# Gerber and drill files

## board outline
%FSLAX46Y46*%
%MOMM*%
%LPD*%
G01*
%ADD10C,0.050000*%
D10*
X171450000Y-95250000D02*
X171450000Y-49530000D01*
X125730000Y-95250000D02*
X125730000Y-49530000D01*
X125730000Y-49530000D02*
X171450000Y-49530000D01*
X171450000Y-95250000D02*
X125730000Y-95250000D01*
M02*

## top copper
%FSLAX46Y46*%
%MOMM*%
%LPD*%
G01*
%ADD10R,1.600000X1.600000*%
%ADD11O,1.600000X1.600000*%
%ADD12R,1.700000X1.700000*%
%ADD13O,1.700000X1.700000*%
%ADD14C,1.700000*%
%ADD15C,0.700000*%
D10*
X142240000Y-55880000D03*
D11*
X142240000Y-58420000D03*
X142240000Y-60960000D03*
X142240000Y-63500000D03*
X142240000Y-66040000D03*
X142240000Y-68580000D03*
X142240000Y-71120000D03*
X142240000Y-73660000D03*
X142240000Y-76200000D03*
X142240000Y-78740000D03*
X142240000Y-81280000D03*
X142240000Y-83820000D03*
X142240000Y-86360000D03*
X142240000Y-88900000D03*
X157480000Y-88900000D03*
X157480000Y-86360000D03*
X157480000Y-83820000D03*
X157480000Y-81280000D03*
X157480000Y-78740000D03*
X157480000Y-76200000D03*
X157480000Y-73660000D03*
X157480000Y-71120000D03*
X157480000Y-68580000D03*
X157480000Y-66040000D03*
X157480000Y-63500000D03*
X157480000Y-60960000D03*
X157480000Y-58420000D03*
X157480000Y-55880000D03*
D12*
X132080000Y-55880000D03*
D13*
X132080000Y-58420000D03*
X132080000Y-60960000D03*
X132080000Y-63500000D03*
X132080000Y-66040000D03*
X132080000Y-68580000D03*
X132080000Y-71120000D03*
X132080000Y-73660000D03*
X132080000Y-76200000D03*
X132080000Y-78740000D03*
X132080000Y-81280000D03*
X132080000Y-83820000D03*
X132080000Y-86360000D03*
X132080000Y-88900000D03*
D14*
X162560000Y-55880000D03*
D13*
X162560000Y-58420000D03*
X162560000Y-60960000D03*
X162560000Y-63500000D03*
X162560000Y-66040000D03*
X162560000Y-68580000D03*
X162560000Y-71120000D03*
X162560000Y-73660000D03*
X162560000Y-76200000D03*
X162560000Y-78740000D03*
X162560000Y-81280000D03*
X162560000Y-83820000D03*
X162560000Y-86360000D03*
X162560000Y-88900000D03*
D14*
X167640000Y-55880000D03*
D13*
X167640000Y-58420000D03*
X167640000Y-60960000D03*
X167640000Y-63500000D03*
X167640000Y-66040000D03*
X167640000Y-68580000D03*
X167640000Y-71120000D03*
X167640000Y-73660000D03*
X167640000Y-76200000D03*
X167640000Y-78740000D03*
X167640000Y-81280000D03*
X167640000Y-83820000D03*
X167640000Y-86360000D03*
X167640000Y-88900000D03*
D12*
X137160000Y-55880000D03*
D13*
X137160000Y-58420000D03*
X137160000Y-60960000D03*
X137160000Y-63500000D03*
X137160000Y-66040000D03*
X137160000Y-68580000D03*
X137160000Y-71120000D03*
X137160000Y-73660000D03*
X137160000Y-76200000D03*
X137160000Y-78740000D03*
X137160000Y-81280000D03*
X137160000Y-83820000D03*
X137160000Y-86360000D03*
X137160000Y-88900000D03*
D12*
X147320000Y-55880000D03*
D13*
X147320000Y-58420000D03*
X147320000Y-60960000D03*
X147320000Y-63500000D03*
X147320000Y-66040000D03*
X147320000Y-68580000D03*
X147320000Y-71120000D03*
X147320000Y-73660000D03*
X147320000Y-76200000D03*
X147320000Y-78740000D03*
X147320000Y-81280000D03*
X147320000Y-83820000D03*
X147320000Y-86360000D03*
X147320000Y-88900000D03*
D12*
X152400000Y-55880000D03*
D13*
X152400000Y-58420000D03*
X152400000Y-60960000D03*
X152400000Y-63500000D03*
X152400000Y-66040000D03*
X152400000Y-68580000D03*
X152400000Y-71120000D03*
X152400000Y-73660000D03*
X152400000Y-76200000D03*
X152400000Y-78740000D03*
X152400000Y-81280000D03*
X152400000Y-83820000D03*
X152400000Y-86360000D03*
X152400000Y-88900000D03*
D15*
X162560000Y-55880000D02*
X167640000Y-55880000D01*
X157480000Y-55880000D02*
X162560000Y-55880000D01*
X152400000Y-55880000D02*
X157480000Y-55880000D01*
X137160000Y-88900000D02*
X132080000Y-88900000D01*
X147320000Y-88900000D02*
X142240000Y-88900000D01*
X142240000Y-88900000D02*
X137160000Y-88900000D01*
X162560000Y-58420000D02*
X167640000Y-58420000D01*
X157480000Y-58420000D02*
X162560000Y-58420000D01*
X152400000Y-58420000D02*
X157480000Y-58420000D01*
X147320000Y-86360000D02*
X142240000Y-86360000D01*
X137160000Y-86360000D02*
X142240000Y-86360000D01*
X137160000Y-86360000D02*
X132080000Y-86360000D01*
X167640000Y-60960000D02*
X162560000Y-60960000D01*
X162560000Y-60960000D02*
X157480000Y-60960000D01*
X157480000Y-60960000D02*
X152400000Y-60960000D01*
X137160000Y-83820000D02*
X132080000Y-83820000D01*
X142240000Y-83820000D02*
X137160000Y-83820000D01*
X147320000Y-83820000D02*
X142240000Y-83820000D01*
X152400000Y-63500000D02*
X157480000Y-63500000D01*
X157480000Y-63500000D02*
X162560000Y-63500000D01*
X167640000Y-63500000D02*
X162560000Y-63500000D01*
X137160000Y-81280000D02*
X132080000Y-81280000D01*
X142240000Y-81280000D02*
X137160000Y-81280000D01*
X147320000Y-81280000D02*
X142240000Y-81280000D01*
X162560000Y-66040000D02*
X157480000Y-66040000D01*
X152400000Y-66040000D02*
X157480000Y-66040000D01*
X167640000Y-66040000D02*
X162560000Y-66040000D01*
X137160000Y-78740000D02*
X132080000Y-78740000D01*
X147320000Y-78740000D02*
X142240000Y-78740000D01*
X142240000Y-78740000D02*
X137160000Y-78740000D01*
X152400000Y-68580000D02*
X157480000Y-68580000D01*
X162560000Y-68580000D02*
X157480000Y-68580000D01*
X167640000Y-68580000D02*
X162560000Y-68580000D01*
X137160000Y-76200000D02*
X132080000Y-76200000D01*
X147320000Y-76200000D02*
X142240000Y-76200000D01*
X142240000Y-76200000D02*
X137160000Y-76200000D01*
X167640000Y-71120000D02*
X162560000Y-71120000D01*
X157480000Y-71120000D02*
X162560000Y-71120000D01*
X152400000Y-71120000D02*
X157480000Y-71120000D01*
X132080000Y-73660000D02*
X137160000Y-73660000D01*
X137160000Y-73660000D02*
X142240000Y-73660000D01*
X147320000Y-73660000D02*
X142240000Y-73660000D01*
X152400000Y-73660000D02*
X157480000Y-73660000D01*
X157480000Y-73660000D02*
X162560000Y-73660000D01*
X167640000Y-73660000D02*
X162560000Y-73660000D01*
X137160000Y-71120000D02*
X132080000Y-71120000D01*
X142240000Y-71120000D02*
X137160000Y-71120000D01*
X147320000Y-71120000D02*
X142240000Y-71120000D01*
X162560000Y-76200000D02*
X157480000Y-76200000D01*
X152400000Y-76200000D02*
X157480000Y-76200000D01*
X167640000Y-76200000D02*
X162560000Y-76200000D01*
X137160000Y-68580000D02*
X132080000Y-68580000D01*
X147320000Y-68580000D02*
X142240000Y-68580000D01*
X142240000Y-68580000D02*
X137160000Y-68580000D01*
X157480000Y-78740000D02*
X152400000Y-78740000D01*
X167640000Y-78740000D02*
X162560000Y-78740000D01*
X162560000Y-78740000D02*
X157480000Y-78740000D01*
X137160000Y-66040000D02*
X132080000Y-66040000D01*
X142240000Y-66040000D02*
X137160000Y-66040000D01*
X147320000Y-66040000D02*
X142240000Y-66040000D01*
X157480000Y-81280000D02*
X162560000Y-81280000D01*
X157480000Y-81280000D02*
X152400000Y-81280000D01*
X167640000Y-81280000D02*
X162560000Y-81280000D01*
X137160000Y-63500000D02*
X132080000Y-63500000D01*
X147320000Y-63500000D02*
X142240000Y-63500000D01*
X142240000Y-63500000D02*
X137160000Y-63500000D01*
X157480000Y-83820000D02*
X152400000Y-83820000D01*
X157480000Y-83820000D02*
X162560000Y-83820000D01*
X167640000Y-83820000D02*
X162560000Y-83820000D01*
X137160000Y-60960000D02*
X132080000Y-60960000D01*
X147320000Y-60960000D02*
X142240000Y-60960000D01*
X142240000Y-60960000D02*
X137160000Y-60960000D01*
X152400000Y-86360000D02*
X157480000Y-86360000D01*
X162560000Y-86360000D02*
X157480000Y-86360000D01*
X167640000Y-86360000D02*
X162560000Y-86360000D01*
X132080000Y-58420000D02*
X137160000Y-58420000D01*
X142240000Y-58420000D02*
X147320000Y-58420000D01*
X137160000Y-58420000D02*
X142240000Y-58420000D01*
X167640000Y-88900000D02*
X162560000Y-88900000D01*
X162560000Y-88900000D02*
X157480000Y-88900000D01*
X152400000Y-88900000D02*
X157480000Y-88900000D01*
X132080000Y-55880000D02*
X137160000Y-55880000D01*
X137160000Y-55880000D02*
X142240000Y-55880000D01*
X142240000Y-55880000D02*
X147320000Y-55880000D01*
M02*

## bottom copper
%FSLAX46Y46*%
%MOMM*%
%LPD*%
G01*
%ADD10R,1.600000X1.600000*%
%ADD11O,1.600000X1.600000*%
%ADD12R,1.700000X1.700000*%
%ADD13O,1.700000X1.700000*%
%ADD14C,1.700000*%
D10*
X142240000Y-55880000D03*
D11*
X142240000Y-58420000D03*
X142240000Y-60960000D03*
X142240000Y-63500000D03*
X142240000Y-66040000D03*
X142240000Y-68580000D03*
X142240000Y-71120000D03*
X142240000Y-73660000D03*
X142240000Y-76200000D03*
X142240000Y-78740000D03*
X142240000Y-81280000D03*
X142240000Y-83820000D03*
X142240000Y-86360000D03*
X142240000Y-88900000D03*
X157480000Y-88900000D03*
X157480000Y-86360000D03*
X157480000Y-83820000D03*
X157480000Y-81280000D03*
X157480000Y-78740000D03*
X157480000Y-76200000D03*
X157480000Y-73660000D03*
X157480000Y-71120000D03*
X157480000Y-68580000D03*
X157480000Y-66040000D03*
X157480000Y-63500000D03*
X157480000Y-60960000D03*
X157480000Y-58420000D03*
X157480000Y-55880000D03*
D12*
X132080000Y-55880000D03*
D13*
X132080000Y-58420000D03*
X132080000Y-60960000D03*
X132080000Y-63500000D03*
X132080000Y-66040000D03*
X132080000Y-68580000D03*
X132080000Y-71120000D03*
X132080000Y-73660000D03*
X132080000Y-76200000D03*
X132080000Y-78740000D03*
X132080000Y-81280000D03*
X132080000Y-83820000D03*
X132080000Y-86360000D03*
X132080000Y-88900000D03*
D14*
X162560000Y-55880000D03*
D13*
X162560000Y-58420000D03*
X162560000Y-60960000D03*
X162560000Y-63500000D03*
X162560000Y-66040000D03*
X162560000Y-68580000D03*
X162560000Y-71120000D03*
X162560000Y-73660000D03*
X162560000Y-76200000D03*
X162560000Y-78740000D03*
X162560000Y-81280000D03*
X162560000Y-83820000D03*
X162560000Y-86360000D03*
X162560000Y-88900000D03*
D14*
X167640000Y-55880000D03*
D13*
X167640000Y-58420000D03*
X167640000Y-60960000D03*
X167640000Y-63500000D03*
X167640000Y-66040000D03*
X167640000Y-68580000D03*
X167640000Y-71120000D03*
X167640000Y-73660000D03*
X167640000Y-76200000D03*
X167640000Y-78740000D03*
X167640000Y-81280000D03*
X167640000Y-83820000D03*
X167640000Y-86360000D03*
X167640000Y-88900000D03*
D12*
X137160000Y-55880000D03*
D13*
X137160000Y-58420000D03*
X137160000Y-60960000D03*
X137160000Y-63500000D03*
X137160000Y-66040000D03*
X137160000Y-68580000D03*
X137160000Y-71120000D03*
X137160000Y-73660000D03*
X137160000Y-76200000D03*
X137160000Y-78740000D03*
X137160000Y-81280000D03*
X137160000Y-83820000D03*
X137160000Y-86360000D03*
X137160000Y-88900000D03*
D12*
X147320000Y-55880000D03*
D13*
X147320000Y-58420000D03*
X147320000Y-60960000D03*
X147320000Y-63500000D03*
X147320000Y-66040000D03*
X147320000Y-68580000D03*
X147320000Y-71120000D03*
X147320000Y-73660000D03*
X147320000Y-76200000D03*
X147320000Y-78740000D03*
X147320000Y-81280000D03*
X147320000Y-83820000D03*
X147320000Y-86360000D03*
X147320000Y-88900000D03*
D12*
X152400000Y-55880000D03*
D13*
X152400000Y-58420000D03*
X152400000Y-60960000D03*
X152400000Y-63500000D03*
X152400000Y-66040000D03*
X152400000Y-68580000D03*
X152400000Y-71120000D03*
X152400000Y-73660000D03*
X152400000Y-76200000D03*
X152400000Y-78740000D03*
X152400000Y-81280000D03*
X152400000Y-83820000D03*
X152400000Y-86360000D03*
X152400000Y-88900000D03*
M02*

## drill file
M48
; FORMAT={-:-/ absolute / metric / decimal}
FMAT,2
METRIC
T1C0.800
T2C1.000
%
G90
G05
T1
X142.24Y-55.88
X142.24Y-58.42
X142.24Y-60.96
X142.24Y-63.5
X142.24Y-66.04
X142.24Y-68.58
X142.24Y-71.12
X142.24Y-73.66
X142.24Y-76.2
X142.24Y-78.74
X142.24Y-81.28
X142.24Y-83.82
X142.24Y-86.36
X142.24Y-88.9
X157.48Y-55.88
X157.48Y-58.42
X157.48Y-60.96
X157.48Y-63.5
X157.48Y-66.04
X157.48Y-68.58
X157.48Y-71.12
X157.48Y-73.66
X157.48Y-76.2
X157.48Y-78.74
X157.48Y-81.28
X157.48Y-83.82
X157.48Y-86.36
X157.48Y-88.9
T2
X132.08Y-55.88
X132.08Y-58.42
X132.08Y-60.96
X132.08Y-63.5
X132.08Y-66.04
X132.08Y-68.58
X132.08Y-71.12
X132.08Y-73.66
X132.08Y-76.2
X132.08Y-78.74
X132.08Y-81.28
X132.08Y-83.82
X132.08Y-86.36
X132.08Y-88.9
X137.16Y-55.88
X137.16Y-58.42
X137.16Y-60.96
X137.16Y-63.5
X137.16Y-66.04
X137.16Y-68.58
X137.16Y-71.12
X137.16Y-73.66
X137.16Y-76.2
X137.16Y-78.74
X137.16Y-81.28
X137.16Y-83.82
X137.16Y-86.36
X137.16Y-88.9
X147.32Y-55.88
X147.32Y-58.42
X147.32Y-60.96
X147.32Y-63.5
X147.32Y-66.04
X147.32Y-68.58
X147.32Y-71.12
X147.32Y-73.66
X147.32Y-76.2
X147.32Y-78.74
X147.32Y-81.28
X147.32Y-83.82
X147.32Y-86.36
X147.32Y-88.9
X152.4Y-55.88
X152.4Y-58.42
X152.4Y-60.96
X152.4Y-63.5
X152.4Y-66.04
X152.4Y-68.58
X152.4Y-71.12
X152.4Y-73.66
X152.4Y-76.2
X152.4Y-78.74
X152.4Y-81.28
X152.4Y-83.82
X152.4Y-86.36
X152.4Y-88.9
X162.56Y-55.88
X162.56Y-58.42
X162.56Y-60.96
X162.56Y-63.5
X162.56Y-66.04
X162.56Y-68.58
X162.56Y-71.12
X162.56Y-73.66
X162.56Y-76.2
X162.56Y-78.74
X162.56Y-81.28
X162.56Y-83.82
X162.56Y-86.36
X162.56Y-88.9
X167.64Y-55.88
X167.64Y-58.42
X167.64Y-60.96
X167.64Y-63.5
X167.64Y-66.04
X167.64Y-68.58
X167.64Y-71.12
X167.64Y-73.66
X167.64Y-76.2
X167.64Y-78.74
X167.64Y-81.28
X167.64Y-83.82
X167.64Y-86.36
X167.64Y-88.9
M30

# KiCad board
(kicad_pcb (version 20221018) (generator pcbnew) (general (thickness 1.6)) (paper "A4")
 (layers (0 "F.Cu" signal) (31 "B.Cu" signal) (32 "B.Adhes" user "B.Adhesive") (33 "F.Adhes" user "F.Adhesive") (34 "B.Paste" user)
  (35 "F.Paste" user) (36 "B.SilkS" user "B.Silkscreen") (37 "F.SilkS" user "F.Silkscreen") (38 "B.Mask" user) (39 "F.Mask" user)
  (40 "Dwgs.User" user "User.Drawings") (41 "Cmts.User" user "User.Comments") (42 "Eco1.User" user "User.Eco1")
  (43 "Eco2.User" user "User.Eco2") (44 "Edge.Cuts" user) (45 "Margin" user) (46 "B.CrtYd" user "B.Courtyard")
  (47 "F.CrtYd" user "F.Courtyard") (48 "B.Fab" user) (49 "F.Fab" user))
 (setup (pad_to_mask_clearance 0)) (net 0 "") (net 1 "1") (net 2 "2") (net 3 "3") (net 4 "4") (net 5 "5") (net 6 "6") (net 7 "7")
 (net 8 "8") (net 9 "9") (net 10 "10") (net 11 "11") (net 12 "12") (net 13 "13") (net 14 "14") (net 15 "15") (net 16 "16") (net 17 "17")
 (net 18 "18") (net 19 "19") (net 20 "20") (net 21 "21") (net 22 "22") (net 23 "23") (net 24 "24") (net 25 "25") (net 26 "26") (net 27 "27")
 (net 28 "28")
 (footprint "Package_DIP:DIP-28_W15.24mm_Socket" (layer "F.Cu") (at 142.24 55.88)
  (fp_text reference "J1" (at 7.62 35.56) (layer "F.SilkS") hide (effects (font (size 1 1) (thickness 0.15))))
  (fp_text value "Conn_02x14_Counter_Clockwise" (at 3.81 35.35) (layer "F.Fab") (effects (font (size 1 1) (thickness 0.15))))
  (pad "1" thru_hole rect (at 0 0) (size 1.6 1.6) (drill 0.8) (layers "*.Cu" "*.Mask") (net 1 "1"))
  (pad "2" thru_hole oval (at 0 2.54) (size 1.6 1.6) (drill 0.8) (layers "*.Cu" "*.Mask") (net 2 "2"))
  (pad "3" thru_hole oval (at 0 5.08) (size 1.6 1.6) (drill 0.8) (layers "*.Cu" "*.Mask") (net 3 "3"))
  (pad "4" thru_hole oval (at 0 7.62) (size 1.6 1.6) (drill 0.8) (layers "*.Cu" "*.Mask") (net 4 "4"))
  (pad "5" thru_hole oval (at 0 10.16) (size 1.6 1.6) (drill 0.8) (layers "*.Cu" "*.Mask") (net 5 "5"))
  (pad "6" thru_hole oval (at 0 12.7) (size 1.6 1.6) (drill 0.8) (layers "*.Cu" "*.Mask") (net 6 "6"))
  (pad "7" thru_hole oval (at 0 15.24) (size 1.6 1.6) (drill 0.8) (layers "*.Cu" "*.Mask") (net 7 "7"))
  (pad "8" thru_hole oval (at 0 17.78) (size 1.6 1.6) (drill 0.8) (layers "*.Cu" "*.Mask") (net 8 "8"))
  (pad "9" thru_hole oval (at 0 20.32) (size 1.6 1.6) (drill 0.8) (layers "*.Cu" "*.Mask") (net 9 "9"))
  (pad "10" thru_hole oval (at 0 22.86) (size 1.6 1.6) (drill 0.8) (layers "*.Cu" "*.Mask") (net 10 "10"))
  (pad "11" thru_hole oval (at 0 25.4) (size 1.6 1.6) (drill 0.8) (layers "*.Cu" "*.Mask") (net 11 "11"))
  (pad "12" thru_hole oval (at 0 27.94) (size 1.6 1.6) (drill 0.8) (layers "*.Cu" "*.Mask") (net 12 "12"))
  (pad "13" thru_hole oval (at 0 30.48) (size 1.6 1.6) (drill 0.8) (layers "*.Cu" "*.Mask") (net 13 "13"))
  (pad "14" thru_hole oval (at 0 33.02) (size 1.6 1.6) (drill 0.8) (layers "*.Cu" "*.Mask") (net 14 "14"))
  (pad "15" thru_hole oval (at 15.24 33.02) (size 1.6 1.6) (drill 0.8) (layers "*.Cu" "*.Mask") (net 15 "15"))
  (pad "16" thru_hole oval (at 15.24 30.48) (size 1.6 1.6) (drill 0.8) (layers "*.Cu" "*.Mask") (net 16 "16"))
  (pad "17" thru_hole oval (at 15.24 27.94) (size 1.6 1.6) (drill 0.8) (layers "*.Cu" "*.Mask") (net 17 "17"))
  (pad "18" thru_hole oval (at 15.24 25.4) (size 1.6 1.6) (drill 0.8) (layers "*.Cu" "*.Mask") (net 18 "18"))
  (pad "19" thru_hole oval (at 15.24 22.86) (size 1.6 1.6) (drill 0.8) (layers "*.Cu" "*.Mask") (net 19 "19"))
  (pad "20" thru_hole oval (at 15.24 20.32) (size 1.6 1.6) (drill 0.8) (layers "*.Cu" "*.Mask") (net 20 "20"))
  (pad "21" thru_hole oval (at 15.24 17.78) (size 1.6 1.6) (drill 0.8) (layers "*.Cu" "*.Mask") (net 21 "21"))
  (pad "22" thru_hole oval (at 15.24 15.24) (size 1.6 1.6) (drill 0.8) (layers "*.Cu" "*.Mask") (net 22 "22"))
  (pad "23" thru_hole oval (at 15.24 12.7) (size 1.6 1.6) (drill 0.8) (layers "*.Cu" "*.Mask") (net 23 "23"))
  (pad "24" thru_hole oval (at 15.24 10.16) (size 1.6 1.6) (drill 0.8) (layers "*.Cu" "*.Mask") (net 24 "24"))
  (pad "25" thru_hole oval (at 15.24 7.62) (size 1.6 1.6) (drill 0.8) (layers "*.Cu" "*.Mask") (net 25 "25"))
  (pad "26" thru_hole oval (at 15.24 5.08) (size 1.6 1.6) (drill 0.8) (layers "*.Cu" "*.Mask") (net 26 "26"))
  (pad "27" thru_hole oval (at 15.24 2.54) (size 1.6 1.6) (drill 0.8) (layers "*.Cu" "*.Mask") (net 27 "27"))
  (pad "28" thru_hole oval (at 15.24 0) (size 1.6 1.6) (drill 0.8) (layers "*.Cu" "*.Mask") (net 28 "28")))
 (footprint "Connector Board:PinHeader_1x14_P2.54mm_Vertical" (layer "F.Cu") (at 132.08 55.88)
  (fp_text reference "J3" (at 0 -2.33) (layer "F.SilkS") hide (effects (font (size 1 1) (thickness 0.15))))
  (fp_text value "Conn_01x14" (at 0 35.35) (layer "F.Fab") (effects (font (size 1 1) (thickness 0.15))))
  (pad "1" thru_hole rect (at 0 0) (size 1.7 1.7) (drill 1) (layers "*.Cu" "*.Mask") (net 1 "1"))
  (pad "2" thru_hole oval (at 0 2.54) (size 1.7 1.7) (drill 1) (layers "*.Cu" "*.Mask") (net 2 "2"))
  (pad "3" thru_hole oval (at 0 5.08) (size 1.7 1.7) (drill 1) (layers "*.Cu" "*.Mask") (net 3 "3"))
  (pad "4" thru_hole oval (at 0 7.62) (size 1.7 1.7) (drill 1) (layers "*.Cu" "*.Mask") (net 4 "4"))
  (pad "5" thru_hole oval (at 0 10.16) (size 1.7 1.7) (drill 1) (layers "*.Cu" "*.Mask") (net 5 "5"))
  (pad "6" thru_hole oval (at 0 12.7) (size 1.7 1.7) (drill 1) (layers "*.Cu" "*.Mask") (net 6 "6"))
  (pad "7" thru_hole oval (at 0 15.24) (size 1.7 1.7) (drill 1) (layers "*.Cu" "*.Mask") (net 7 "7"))
  (pad "8" thru_hole oval (at 0 17.78) (size 1.7 1.7) (drill 1) (layers "*.Cu" "*.Mask") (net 8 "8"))
  (pad "9" thru_hole oval (at 0 20.32) (size 1.7 1.7) (drill 1) (layers "*.Cu" "*.Mask") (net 9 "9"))
  (pad "10" thru_hole oval (at 0 22.86) (size 1.7 1.7) (drill 1) (layers "*.Cu" "*.Mask") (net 10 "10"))
  (pad "11" thru_hole oval (at 0 25.4) (size 1.7 1.7) (drill 1) (layers "*.Cu" "*.Mask") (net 11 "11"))
  (pad "12" thru_hole oval (at 0 27.94) (size 1.7 1.7) (drill 1) (layers "*.Cu" "*.Mask") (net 12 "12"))
  (pad "13" thru_hole oval (at 0 30.48) (size 1.7 1.7) (drill 1) (layers "*.Cu" "*.Mask") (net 13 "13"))
  (pad "14" thru_hole oval (at 0 33.02) (size 1.7 1.7) (drill 1) (layers "*.Cu" "*.Mask") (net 14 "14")))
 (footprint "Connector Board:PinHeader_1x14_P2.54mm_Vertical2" (layer "F.Cu") (at 162.56 55.88)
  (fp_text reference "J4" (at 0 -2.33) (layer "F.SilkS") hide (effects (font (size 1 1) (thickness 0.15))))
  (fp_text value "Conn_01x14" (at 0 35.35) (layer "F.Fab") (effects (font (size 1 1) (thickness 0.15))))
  (pad "1" thru_hole circle (at 0 0) (size 1.7 1.7) (drill 1) (layers "*.Cu" "*.Mask") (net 28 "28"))
  (pad "2" thru_hole oval (at 0 2.54) (size 1.7 1.7) (drill 1) (layers "*.Cu" "*.Mask") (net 27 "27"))
  (pad "3" thru_hole oval (at 0 5.08) (size 1.7 1.7) (drill 1) (layers "*.Cu" "*.Mask") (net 26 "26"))
  (pad "4" thru_hole oval (at 0 7.62) (size 1.7 1.7) (drill 1) (layers "*.Cu" "*.Mask") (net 25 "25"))
  (pad "5" thru_hole oval (at 0 10.16) (size 1.7 1.7) (drill 1) (layers "*.Cu" "*.Mask") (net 24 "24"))
  (pad "6" thru_hole oval (at 0 12.7) (size 1.7 1.7) (drill 1) (layers "*.Cu" "*.Mask") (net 23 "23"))
  (pad "7" thru_hole oval (at 0 15.24) (size 1.7 1.7) (drill 1) (layers "*.Cu" "*.Mask") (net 22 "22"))
  (pad "8" thru_hole oval (at 0 17.78) (size 1.7 1.7) (drill 1) (layers "*.Cu" "*.Mask") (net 21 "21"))
  (pad "9" thru_hole oval (at 0 20.32) (size 1.7 1.7) (drill 1) (layers "*.Cu" "*.Mask") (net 20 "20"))
  (pad "10" thru_hole oval (at 0 22.86) (size 1.7 1.7) (drill 1) (layers "*.Cu" "*.Mask") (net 19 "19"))
  (pad "11" thru_hole oval (at 0 25.4) (size 1.7 1.7) (drill 1) (layers "*.Cu" "*.Mask") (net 18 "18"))
  (pad "12" thru_hole oval (at 0 27.94) (size 1.7 1.7) (drill 1) (layers "*.Cu" "*.Mask") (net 17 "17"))
  (pad "13" thru_hole oval (at 0 30.48) (size 1.7 1.7) (drill 1) (layers "*.Cu" "*.Mask") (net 16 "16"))
  (pad "14" thru_hole oval (at 0 33.02) (size 1.7 1.7) (drill 1) (layers "*.Cu" "*.Mask") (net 15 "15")))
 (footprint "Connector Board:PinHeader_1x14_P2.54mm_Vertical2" (layer "F.Cu") (at 167.64 55.88)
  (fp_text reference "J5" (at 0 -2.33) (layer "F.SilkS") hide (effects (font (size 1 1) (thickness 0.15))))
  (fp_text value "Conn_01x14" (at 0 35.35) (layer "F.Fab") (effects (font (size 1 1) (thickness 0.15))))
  (pad "1" thru_hole circle (at 0 0) (size 1.7 1.7) (drill 1) (layers "*.Cu" "*.Mask") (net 28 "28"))
  (pad "2" thru_hole oval (at 0 2.54) (size 1.7 1.7) (drill 1) (layers "*.Cu" "*.Mask") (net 27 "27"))
  (pad "3" thru_hole oval (at 0 5.08) (size 1.7 1.7) (drill 1) (layers "*.Cu" "*.Mask") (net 26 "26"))
  (pad "4" thru_hole oval (at 0 7.62) (size 1.7 1.7) (drill 1) (layers "*.Cu" "*.Mask") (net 25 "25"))
  (pad "5" thru_hole oval (at 0 10.16) (size 1.7 1.7) (drill 1) (layers "*.Cu" "*.Mask") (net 24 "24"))
  (pad "6" thru_hole oval (at 0 12.7) (size 1.7 1.7) (drill 1) (layers "*.Cu" "*.Mask") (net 23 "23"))
  (pad "7" thru_hole oval (at 0 15.24) (size 1.7 1.7) (drill 1) (layers "*.Cu" "*.Mask") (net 22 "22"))
  (pad "8" thru_hole oval (at 0 17.78) (size 1.7 1.7) (drill 1) (layers "*.Cu" "*.Mask") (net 21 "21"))
  (pad "9" thru_hole oval (at 0 20.32) (size 1.7 1.7) (drill 1) (layers "*.Cu" "*.Mask") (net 20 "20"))
  (pad "10" thru_hole oval (at 0 22.86) (size 1.7 1.7) (drill 1) (layers "*.Cu" "*.Mask") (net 19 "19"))
  (pad "11" thru_hole oval (at 0 25.4) (size 1.7 1.7) (drill 1) (layers "*.Cu" "*.Mask") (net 18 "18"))
  (pad "12" thru_hole oval (at 0 27.94) (size 1.7 1.7) (drill 1) (layers "*.Cu" "*.Mask") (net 17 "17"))
  (pad "13" thru_hole oval (at 0 30.48) (size 1.7 1.7) (drill 1) (layers "*.Cu" "*.Mask") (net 16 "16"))
  (pad "14" thru_hole oval (at 0 33.02) (size 1.7 1.7) (drill 1) (layers "*.Cu" "*.Mask") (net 15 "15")))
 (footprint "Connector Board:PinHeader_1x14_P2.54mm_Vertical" (layer "F.Cu") (at 137.16 55.88)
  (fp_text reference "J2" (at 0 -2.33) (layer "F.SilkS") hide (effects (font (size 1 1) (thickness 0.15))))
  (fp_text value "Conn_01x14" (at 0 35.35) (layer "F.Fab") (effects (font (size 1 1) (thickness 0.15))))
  (pad "1" thru_hole rect (at 0 0) (size 1.7 1.7) (drill 1) (layers "*.Cu" "*.Mask") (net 1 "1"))
  (pad "2" thru_hole oval (at 0 2.54) (size 1.7 1.7) (drill 1) (layers "*.Cu" "*.Mask") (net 2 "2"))
  (pad "3" thru_hole oval (at 0 5.08) (size 1.7 1.7) (drill 1) (layers "*.Cu" "*.Mask") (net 3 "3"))
  (pad "4" thru_hole oval (at 0 7.62) (size 1.7 1.7) (drill 1) (layers "*.Cu" "*.Mask") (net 4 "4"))
  (pad "5" thru_hole oval (at 0 10.16) (size 1.7 1.7) (drill 1) (layers "*.Cu" "*.Mask") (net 5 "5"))
  (pad "6" thru_hole oval (at 0 12.7) (size 1.7 1.7) (drill 1) (layers "*.Cu" "*.Mask") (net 6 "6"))
  (pad "7" thru_hole oval (at 0 15.24) (size 1.7 1.7) (drill 1) (layers "*.Cu" "*.Mask") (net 7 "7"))
  (pad "8" thru_hole oval (at 0 17.78) (size 1.7 1.7) (drill 1) (layers "*.Cu" "*.Mask") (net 8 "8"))
  (pad "9" thru_hole oval (at 0 20.32) (size 1.7 1.7) (drill 1) (layers "*.Cu" "*.Mask") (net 9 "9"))
  (pad "10" thru_hole oval (at 0 22.86) (size 1.7 1.7) (drill 1) (layers "*.Cu" "*.Mask") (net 10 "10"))
  (pad "11" thru_hole oval (at 0 25.4) (size 1.7 1.7) (drill 1) (layers "*.Cu" "*.Mask") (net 11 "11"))
  (pad "12" thru_hole oval (at 0 27.94) (size 1.7 1.7) (drill 1) (layers "*.Cu" "*.Mask") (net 12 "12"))
  (pad "13" thru_hole oval (at 0 30.48) (size 1.7 1.7) (drill 1) (layers "*.Cu" "*.Mask") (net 13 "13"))
  (pad "14" thru_hole oval (at 0 33.02) (size 1.7 1.7) (drill 1) (layers "*.Cu" "*.Mask") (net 14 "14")))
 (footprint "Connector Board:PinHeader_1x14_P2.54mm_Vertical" (layer "F.Cu") (at 147.32 55.88)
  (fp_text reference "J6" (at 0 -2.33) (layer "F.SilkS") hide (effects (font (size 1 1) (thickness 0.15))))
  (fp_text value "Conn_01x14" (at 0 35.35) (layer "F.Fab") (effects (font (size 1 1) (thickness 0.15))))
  (pad "1" thru_hole rect (at 0 0) (size 1.7 1.7) (drill 1) (layers "*.Cu" "*.Mask") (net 1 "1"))
  (pad "2" thru_hole oval (at 0 2.54) (size 1.7 1.7) (drill 1) (layers "*.Cu" "*.Mask") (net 2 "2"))
  (pad "3" thru_hole oval (at 0 5.08) (size 1.7 1.7) (drill 1) (layers "*.Cu" "*.Mask") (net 3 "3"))
  (pad "4" thru_hole oval (at 0 7.62) (size 1.7 1.7) (drill 1) (layers "*.Cu" "*.Mask") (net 4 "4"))
  (pad "5" thru_hole oval (at 0 10.16) (size 1.7 1.7) (drill 1) (layers "*.Cu" "*.Mask") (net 5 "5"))
  (pad "6" thru_hole oval (at 0 12.7) (size 1.7 1.7) (drill 1) (layers "*.Cu" "*.Mask") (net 6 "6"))
  (pad "7" thru_hole oval (at 0 15.24) (size 1.7 1.7) (drill 1) (layers "*.Cu" "*.Mask") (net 7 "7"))
  (pad "8" thru_hole oval (at 0 17.78) (size 1.7 1.7) (drill 1) (layers "*.Cu" "*.Mask") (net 8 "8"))
  (pad "9" thru_hole oval (at 0 20.32) (size 1.7 1.7) (drill 1) (layers "*.Cu" "*.Mask") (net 9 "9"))
  (pad "10" thru_hole oval (at 0 22.86) (size 1.7 1.7) (drill 1) (layers "*.Cu" "*.Mask") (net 10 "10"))
  (pad "11" thru_hole oval (at 0 25.4) (size 1.7 1.7) (drill 1) (layers "*.Cu" "*.Mask") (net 11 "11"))
  (pad "12" thru_hole oval (at 0 27.94) (size 1.7 1.7) (drill 1) (layers "*.Cu" "*.Mask") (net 12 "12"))
  (pad "13" thru_hole oval (at 0 30.48) (size 1.7 1.7) (drill 1) (layers "*.Cu" "*.Mask") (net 13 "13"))
  (pad "14" thru_hole oval (at 0 33.02) (size 1.7 1.7) (drill 1) (layers "*.Cu" "*.Mask") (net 14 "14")))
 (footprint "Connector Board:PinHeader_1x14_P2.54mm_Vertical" (layer "F.Cu") (at 152.4 55.88)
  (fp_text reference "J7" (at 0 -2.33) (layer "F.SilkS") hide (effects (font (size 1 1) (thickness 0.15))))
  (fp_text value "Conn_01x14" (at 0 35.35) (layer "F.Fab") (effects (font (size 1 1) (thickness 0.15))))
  (pad "1" thru_hole rect (at 0 0) (size 1.7 1.7) (drill 1) (layers "*.Cu" "*.Mask") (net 28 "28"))
  (pad "2" thru_hole oval (at 0 2.54) (size 1.7 1.7) (drill 1) (layers "*.Cu" "*.Mask") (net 27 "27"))
  (pad "3" thru_hole oval (at 0 5.08) (size 1.7 1.7) (drill 1) (layers "*.Cu" "*.Mask") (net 26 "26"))
  (pad "4" thru_hole oval (at 0 7.62) (size 1.7 1.7) (drill 1) (layers "*.Cu" "*.Mask") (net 25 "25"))
  (pad "5" thru_hole oval (at 0 10.16) (size 1.7 1.7) (drill 1) (layers "*.Cu" "*.Mask") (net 24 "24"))
  (pad "6" thru_hole oval (at 0 12.7) (size 1.7 1.7) (drill 1) (layers "*.Cu" "*.Mask") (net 23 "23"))
  (pad "7" thru_hole oval (at 0 15.24) (size 1.7 1.7) (drill 1) (layers "*.Cu" "*.Mask") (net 22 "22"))
  (pad "8" thru_hole oval (at 0 17.78) (size 1.7 1.7) (drill 1) (layers "*.Cu" "*.Mask") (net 21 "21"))
  (pad "9" thru_hole oval (at 0 20.32) (size 1.7 1.7) (drill 1) (layers "*.Cu" "*.Mask") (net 20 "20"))
  (pad "10" thru_hole oval (at 0 22.86) (size 1.7 1.7) (drill 1) (layers "*.Cu" "*.Mask") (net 19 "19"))
  (pad "11" thru_hole oval (at 0 25.4) (size 1.7 1.7) (drill 1) (layers "*.Cu" "*.Mask") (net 18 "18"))
  (pad "12" thru_hole oval (at 0 27.94) (size 1.7 1.7) (drill 1) (layers "*.Cu" "*.Mask") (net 17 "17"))
  (pad "13" thru_hole oval (at 0 30.48) (size 1.7 1.7) (drill 1) (layers "*.Cu" "*.Mask") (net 16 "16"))
  (pad "14" thru_hole oval (at 0 33.02) (size 1.7 1.7) (drill 1) (layers "*.Cu" "*.Mask") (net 15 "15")))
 (gr_line (start 171.45 95.25) (end 171.45 49.53) (stroke (width 0.05) (type solid)) (layer "Edge.Cuts"))
 (gr_line (start 125.73 95.25) (end 125.73 49.53) (stroke (width 0.05) (type solid)) (layer "Edge.Cuts"))
 (gr_line (start 125.73 49.53) (end 171.45 49.53) (stroke (width 0.05) (type solid)) (layer "Edge.Cuts"))
 (gr_line (start 171.45 95.25) (end 125.73 95.25) (stroke (width 0.05) (type solid)) (layer "Edge.Cuts"))
 (segment (start 162.56 55.88) (end 167.64 55.88) (width 0.7) (layer "F.Cu") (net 28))
 (segment (start 157.48 55.88) (end 162.56 55.88) (width 0.7) (layer "F.Cu") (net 28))
 (segment (start 152.4 55.88) (end 157.48 55.88) (width 0.7) (layer "F.Cu") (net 28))
 (segment (start 137.16 88.9) (end 132.08 88.9) (width 0.7) (layer "F.Cu") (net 14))
 (segment (start 147.32 88.9) (end 142.24 88.9) (width 0.7) (layer "F.Cu") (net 14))
 (segment (start 142.24 88.9) (end 137.16 88.9) (width 0.7) (layer "F.Cu") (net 14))
 (segment (start 162.56 58.42) (end 167.64 58.42) (width 0.7) (layer "F.Cu") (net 27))
 (segment (start 157.48 58.42) (end 162.56 58.42) (width 0.7) (layer "F.Cu") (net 27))
 (segment (start 152.4 58.42) (end 157.48 58.42) (width 0.7) (layer "F.Cu") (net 27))
 (segment (start 147.32 86.36) (end 142.24 86.36) (width 0.7) (layer "F.Cu") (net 13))
 (segment (start 137.16 86.36) (end 142.24 86.36) (width 0.7) (layer "F.Cu") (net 13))
 (segment (start 137.16 86.36) (end 132.08 86.36) (width 0.7) (layer "F.Cu") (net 13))
 (segment (start 167.64 60.96) (end 162.56 60.96) (width 0.7) (layer "F.Cu") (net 26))
 (segment (start 162.56 60.96) (end 157.48 60.96) (width 0.7) (layer "F.Cu") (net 26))
 (segment (start 157.48 60.96) (end 152.4 60.96) (width 0.7) (layer "F.Cu") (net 26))
 (segment (start 137.16 83.82) (end 132.08 83.82) (width 0.7) (layer "F.Cu") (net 12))
 (segment (start 142.24 83.82) (end 137.16 83.82) (width 0.7) (layer "F.Cu") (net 12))
 (segment (start 147.32 83.82) (end 142.24 83.82) (width 0.7) (layer "F.Cu") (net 12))
 (segment (start 152.4 63.5) (end 157.48 63.5) (width 0.7) (layer "F.Cu") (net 25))
 (segment (start 157.48 63.5) (end 162.56 63.5) (width 0.7) (layer "F.Cu") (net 25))
 (segment (start 167.64 63.5) (end 162.56 63.5) (width 0.7) (layer "F.Cu") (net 25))
 (segment (start 137.16 81.28) (end 132.08 81.28) (width 0.7) (layer "F.Cu") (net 11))
 (segment (start 142.24 81.28) (end 137.16 81.28) (width 0.7) (layer "F.Cu") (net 11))
 (segment (start 147.32 81.28) (end 142.24 81.28) (width 0.7) (layer "F.Cu") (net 11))
 (segment (start 162.56 66.04) (end 157.48 66.04) (width 0.7) (layer "F.Cu") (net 24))
 (segment (start 152.4 66.04) (end 157.48 66.04) (width 0.7) (layer "F.Cu") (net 24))
 (segment (start 167.64 66.04) (end 162.56 66.04) (width 0.7) (layer "F.Cu") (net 24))
 (segment (start 137.16 78.74) (end 132.08 78.74) (width 0.7) (layer "F.Cu") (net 10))
 (segment (start 147.32 78.74) (end 142.24 78.74) (width 0.7) (layer "F.Cu") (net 10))
 (segment (start 142.24 78.74) (end 137.16 78.74) (width 0.7) (layer "F.Cu") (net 10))
 (segment (start 152.4 68.58) (end 157.48 68.58) (width 0.7) (layer "F.Cu") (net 23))
 (segment (start 162.56 68.58) (end 157.48 68.58) (width 0.7) (layer "F.Cu") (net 23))
 (segment (start 167.64 68.58) (end 162.56 68.58) (width 0.7) (layer "F.Cu") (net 23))
 (segment (start 137.16 76.2) (end 132.08 76.2) (width 0.7) (layer "F.Cu") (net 9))
 (segment (start 147.32 76.2) (end 142.24 76.2) (width 0.7) (layer "F.Cu") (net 9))
 (segment (start 142.24 76.2) (end 137.16 76.2) (width 0.7) (layer "F.Cu") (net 9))
 (segment (start 167.64 71.12) (end 162.56 71.12) (width 0.7) (layer "F.Cu") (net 22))
 (segment (start 157.48 71.12) (end 162.56 71.12) (width 0.7) (layer "F.Cu") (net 22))
 (segment (start 152.4 71.12) (end 157.48 71.12) (width 0.7) (layer "F.Cu") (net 22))
 (segment (start 132.08 73.66) (end 137.16 73.66) (width 0.7) (layer "F.Cu") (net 8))
 (segment (start 137.16 73.66) (end 142.24 73.66) (width 0.7) (layer "F.Cu") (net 8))
 (segment (start 147.32 73.66) (end 142.24 73.66) (width 0.7) (layer "F.Cu") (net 8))
 (segment (start 152.4 73.66) (end 157.48 73.66) (width 0.7) (layer "F.Cu") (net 21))
 (segment (start 157.48 73.66) (end 162.56 73.66) (width 0.7) (layer "F.Cu") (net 21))
 (segment (start 167.64 73.66) (end 162.56 73.66) (width 0.7) (layer "F.Cu") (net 21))
 (segment (start 137.16 71.12) (end 132.08 71.12) (width 0.7) (layer "F.Cu") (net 7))
 (segment (start 142.24 71.12) (end 137.16 71.12) (width 0.7) (layer "F.Cu") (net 7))
 (segment (start 147.32 71.12) (end 142.24 71.12) (width 0.7) (layer "F.Cu") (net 7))
 (segment (start 162.56 76.2) (end 157.48 76.2) (width 0.7) (layer "F.Cu") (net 20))
 (segment (start 152.4 76.2) (end 157.48 76.2) (width 0.7) (layer "F.Cu") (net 20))
 (segment (start 167.64 76.2) (end 162.56 76.2) (width 0.7) (layer "F.Cu") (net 20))
 (segment (start 137.16 68.58) (end 132.08 68.58) (width 0.7) (layer "F.Cu") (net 6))
 (segment (start 147.32 68.58) (end 142.24 68.58) (width 0.7) (layer "F.Cu") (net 6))
 (segment (start 142.24 68.58) (end 137.16 68.58) (width 0.7) (layer "F.Cu") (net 6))
 (segment (start 157.48 78.74) (end 152.4 78.74) (width 0.7) (layer "F.Cu") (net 19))
 (segment (start 167.64 78.74) (end 162.56 78.74) (width 0.7) (layer "F.Cu") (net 19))
 (segment (start 162.56 78.74) (end 157.48 78.74) (width 0.7) (layer "F.Cu") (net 19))
 (segment (start 137.16 66.04) (end 132.08 66.04) (width 0.7) (layer "F.Cu") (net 5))
 (segment (start 142.24 66.04) (end 137.16 66.04) (width 0.7) (layer "F.Cu") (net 5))
 (segment (start 147.32 66.04) (end 142.24 66.04) (width 0.7) (layer "F.Cu") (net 5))
 (segment (start 157.48 81.28) (end 162.56 81.28) (width 0.7) (layer "F.Cu") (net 18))
 (segment (start 157.48 81.28) (end 152.4 81.28) (width 0.7) (layer "F.Cu") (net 18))
 (segment (start 167.64 81.28) (end 162.56 81.28) (width 0.7) (layer "F.Cu") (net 18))
 (segment (start 137.16 63.5) (end 132.08 63.5) (width 0.7) (layer "F.Cu") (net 4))
 (segment (start 147.32 63.5) (end 142.24 63.5) (width 0.7) (layer "F.Cu") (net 4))
 (segment (start 142.24 63.5) (end 137.16 63.5) (width 0.7) (layer "F.Cu") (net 4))
 (segment (start 157.48 83.82) (end 152.4 83.82) (width 0.7) (layer "F.Cu") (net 17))
 (segment (start 157.48 83.82) (end 162.56 83.82) (width 0.7) (layer "F.Cu") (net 17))
 (segment (start 167.64 83.82) (end 162.56 83.82) (width 0.7) (layer "F.Cu") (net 17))
 (segment (start 137.16 60.96) (end 132.08 60.96) (width 0.7) (layer "F.Cu") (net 3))
 (segment (start 147.32 60.96) (end 142.24 60.96) (width 0.7) (layer "F.Cu") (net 3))
 (segment (start 142.24 60.96) (end 137.16 60.96) (width 0.7) (layer "F.Cu") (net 3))
 (segment (start 152.4 86.36) (end 157.48 86.36) (width 0.7) (layer "F.Cu") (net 16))
 (segment (start 162.56 86.36) (end 157.48 86.36) (width 0.7) (layer "F.Cu") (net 16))
 (segment (start 167.64 86.36) (end 162.56 86.36) (width 0.7) (layer "F.Cu") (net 16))
 (segment (start 132.08 58.42) (end 137.16 58.42) (width 0.7) (layer "F.Cu") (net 2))
 (segment (start 142.24 58.42) (end 147.32 58.42) (width 0.7) (layer "F.Cu") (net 2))
 (segment (start 137.16 58.42) (end 142.24 58.42) (width 0.7) (layer "F.Cu") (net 2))
 (segment (start 167.64 88.9) (end 162.56 88.9) (width 0.7) (layer "F.Cu") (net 15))
 (segment (start 162.56 88.9) (end 157.48 88.9) (width 0.7) (layer "F.Cu") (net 15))
 (segment (start 152.4 88.9) (end 157.48 88.9) (width 0.7) (layer "F.Cu") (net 15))
 (segment (start 132.08 55.88) (end 137.16 55.88) (width 0.7) (layer "F.Cu") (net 1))
 (segment (start 137.16 55.88) (end 142.24 55.88) (width 0.7) (layer "F.Cu") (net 1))
 (segment (start 142.24 55.88) (end 147.32 55.88) (width 0.7) (layer "F.Cu") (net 1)))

